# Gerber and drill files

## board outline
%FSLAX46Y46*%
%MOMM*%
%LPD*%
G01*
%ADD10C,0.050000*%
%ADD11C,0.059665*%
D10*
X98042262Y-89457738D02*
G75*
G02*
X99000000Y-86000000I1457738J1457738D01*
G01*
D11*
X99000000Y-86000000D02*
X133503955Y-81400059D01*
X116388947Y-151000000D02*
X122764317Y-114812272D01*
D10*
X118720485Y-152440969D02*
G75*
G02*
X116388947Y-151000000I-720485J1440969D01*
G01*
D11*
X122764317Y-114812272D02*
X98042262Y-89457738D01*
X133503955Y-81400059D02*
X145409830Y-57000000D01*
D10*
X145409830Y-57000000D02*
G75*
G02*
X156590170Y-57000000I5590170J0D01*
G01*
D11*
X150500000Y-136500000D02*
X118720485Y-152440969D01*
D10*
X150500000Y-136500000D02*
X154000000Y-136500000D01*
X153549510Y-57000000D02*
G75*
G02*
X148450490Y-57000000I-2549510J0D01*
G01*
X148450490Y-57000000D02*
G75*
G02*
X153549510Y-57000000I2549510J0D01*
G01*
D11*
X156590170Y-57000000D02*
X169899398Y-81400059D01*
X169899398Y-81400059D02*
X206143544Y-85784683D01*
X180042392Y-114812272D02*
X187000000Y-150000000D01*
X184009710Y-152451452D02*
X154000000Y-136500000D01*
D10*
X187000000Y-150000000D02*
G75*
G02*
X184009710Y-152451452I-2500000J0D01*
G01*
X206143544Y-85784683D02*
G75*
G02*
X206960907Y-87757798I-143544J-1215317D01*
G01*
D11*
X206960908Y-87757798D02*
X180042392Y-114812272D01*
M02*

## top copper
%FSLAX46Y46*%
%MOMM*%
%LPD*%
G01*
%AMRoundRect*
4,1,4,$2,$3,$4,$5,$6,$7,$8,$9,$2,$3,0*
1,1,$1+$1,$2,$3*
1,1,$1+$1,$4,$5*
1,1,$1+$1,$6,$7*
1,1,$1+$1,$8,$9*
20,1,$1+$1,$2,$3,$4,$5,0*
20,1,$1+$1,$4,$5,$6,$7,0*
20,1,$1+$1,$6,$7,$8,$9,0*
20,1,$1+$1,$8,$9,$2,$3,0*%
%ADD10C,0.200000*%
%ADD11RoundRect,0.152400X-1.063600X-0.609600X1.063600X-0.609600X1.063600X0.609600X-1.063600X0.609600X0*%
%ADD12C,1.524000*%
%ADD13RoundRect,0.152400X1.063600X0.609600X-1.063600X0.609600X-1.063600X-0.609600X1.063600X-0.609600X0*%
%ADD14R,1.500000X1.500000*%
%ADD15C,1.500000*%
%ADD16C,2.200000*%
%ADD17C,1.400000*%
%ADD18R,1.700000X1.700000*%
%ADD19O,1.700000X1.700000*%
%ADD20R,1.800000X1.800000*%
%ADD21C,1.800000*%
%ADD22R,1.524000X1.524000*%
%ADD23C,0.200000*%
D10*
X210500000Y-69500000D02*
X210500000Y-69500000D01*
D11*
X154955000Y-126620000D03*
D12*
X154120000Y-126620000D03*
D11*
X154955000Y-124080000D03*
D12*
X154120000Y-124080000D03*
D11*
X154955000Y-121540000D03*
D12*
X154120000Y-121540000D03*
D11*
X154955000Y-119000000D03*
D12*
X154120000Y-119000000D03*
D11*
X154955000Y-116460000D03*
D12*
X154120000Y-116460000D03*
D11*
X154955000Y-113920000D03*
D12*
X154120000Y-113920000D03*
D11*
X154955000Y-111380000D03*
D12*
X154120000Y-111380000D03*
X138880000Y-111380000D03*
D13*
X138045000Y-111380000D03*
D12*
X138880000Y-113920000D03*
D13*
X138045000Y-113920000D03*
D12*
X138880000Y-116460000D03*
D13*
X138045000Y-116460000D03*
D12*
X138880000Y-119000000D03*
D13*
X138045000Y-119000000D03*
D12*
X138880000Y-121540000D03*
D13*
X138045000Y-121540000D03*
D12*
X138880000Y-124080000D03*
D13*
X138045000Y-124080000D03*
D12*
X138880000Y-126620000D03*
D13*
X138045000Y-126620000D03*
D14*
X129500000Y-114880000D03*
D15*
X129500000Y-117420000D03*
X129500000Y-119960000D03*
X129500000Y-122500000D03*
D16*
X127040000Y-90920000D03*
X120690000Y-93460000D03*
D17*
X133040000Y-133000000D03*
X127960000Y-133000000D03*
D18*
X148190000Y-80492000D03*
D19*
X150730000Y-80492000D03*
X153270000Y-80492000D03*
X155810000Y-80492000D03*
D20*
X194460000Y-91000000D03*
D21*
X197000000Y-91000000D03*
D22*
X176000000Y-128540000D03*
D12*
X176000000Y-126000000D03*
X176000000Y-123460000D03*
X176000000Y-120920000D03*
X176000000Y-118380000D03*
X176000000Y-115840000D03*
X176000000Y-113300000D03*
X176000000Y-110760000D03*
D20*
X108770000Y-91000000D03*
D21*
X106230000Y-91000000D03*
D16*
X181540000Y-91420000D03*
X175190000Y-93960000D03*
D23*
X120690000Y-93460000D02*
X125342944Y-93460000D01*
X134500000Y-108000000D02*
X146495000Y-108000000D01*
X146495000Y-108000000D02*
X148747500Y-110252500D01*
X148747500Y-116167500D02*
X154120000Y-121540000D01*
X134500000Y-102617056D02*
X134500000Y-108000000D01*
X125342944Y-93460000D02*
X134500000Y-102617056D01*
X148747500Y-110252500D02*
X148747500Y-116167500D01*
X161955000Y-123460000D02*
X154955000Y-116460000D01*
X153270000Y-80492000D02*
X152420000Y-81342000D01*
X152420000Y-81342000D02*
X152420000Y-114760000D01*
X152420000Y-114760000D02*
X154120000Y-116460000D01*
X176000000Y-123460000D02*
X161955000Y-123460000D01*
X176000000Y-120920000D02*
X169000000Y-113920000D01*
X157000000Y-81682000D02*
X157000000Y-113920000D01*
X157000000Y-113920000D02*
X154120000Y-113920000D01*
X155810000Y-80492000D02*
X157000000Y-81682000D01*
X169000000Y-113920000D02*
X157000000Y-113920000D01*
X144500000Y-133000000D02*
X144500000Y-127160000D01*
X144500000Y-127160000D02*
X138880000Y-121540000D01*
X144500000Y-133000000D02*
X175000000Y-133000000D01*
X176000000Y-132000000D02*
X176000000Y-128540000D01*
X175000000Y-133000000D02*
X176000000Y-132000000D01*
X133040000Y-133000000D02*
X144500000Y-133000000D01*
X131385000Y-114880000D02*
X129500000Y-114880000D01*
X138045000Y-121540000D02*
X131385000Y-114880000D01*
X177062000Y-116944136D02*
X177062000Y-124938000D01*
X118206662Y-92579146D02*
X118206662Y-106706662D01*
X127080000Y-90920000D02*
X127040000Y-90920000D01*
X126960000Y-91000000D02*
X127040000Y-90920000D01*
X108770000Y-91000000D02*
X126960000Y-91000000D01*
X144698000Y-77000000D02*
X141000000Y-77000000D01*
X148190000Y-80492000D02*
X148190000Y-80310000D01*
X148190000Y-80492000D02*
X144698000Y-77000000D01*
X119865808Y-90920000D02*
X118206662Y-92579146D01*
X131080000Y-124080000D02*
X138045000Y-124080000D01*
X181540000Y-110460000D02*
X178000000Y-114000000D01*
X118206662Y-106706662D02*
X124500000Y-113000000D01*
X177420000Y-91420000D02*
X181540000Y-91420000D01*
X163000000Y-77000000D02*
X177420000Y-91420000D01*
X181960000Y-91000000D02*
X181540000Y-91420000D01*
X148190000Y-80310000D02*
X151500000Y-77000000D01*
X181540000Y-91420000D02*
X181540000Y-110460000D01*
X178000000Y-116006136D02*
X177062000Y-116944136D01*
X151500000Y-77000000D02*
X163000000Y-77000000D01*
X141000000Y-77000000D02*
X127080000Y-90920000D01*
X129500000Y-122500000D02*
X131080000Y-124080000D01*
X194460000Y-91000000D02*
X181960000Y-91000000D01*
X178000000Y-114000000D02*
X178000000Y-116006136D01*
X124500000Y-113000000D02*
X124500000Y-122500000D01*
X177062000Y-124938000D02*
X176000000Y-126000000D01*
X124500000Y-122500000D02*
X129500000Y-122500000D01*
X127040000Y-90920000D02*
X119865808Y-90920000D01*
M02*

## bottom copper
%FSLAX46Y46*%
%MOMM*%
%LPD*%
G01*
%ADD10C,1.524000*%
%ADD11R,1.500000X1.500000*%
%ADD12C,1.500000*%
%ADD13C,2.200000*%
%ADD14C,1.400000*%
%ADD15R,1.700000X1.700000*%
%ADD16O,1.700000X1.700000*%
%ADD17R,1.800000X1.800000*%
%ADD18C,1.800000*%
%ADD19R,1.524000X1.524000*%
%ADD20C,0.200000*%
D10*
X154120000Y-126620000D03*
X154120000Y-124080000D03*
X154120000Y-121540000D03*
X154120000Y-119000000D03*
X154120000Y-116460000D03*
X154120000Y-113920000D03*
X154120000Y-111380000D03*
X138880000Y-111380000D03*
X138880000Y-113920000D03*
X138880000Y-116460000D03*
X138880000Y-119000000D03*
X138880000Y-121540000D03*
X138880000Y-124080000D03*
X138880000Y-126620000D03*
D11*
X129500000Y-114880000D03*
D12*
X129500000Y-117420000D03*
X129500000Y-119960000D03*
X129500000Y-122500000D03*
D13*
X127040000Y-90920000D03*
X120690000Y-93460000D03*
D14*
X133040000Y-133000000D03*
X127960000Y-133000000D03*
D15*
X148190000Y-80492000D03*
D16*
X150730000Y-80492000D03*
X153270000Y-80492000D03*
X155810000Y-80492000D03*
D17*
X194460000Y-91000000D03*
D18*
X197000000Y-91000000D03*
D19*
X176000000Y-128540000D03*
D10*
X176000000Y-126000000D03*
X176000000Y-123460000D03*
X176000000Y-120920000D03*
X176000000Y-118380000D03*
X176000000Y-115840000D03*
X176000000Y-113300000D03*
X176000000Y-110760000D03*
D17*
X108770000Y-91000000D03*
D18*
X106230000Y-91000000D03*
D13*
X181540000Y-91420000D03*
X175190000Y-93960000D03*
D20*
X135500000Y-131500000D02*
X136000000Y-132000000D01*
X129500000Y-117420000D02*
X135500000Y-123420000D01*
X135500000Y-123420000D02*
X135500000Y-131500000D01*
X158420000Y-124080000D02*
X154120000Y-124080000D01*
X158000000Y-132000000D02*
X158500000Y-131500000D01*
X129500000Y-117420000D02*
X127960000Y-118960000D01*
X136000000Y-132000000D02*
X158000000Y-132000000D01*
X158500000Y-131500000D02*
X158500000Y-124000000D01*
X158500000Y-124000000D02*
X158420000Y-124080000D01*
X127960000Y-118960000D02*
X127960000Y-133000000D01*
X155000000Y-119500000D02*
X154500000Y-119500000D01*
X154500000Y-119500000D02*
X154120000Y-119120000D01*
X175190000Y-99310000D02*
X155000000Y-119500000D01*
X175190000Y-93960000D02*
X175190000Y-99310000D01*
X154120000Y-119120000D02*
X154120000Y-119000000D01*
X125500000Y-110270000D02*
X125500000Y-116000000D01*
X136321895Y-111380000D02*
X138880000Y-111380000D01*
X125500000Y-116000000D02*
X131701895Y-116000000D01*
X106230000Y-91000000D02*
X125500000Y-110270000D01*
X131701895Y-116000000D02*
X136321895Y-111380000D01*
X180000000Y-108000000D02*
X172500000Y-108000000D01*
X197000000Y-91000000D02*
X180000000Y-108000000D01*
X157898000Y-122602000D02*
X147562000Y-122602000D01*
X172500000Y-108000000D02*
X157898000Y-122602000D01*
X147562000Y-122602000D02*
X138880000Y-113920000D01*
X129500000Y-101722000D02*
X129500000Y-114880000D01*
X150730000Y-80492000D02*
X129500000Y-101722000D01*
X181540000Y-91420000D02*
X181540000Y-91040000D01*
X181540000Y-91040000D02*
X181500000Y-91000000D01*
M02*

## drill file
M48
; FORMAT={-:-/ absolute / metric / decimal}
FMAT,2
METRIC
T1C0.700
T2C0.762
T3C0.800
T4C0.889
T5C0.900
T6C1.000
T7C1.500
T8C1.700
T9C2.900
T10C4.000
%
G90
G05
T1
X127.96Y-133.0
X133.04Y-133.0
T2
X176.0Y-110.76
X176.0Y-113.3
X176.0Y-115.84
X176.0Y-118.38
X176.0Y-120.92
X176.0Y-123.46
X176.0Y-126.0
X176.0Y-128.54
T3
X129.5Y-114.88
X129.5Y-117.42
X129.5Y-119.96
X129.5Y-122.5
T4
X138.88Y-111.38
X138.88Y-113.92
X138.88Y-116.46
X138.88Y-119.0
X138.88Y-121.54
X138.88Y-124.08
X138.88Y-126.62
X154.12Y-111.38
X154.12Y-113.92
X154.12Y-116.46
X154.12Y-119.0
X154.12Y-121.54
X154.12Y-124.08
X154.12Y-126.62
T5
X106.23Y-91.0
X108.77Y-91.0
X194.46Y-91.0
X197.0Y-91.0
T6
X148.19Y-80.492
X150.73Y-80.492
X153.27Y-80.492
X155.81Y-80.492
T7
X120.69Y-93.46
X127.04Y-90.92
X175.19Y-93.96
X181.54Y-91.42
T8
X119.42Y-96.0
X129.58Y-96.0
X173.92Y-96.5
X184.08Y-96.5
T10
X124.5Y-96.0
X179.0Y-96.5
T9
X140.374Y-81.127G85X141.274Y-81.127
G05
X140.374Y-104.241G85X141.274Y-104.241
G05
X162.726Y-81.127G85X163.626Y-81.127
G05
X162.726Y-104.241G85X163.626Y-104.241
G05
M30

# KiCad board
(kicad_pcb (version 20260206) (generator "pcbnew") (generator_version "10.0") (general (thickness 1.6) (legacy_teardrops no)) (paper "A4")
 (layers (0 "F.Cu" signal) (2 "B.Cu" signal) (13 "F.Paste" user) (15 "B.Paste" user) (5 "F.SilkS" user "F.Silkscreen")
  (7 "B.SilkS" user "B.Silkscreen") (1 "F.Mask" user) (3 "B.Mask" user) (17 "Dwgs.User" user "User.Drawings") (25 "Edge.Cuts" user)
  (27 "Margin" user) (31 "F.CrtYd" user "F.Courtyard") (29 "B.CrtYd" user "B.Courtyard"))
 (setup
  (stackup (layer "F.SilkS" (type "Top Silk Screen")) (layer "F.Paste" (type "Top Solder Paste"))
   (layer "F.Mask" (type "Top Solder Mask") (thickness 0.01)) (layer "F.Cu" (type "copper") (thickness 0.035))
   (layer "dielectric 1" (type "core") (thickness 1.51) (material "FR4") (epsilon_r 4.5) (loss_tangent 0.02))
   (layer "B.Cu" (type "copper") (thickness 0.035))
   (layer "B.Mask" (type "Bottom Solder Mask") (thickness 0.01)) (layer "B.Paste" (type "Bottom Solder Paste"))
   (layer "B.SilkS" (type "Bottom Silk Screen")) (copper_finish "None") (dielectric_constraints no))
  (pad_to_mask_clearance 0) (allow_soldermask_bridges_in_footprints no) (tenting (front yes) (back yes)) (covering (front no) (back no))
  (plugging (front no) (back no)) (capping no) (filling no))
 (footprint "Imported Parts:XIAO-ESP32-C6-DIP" (layer "F.Cu") (at 146.5 119 -90)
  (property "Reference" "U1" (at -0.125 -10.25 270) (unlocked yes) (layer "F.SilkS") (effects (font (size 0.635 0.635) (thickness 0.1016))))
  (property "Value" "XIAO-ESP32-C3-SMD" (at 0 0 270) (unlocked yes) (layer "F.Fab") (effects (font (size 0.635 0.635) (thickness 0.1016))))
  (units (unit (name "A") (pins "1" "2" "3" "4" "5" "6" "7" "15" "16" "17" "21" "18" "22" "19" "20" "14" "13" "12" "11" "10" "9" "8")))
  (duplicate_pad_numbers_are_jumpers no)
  (pad "1" smd roundrect (at 7.62 -8.455) (size 2.432 1.524) (layers "F.Cu" "F.Mask") (roundrect_rratio 0.1)
   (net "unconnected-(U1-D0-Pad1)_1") (thermal_bridge_angle 45))
  (pad "1" thru_hole circle (at 7.62 -7.62) (size 1.524 1.524) (drill 0.889) (layers "*.Cu" "*.Mask") (remove_unused_layers no)
   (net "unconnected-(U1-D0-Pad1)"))
  (pad "2" smd roundrect (at 5.08 -8.455) (size 2.432 1.524) (layers "F.Cu" "F.Mask") (roundrect_rratio 0.1) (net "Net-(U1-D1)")
   (thermal_bridge_angle 45))
  (pad "2" thru_hole circle (at 5.08 -7.62) (size 1.524 1.524) (drill 0.889) (layers "*.Cu" "*.Mask") (remove_unused_layers no)
   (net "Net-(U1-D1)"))
  (pad "3" smd roundrect (at 2.54 -8.455) (size 2.432 1.524) (layers "F.Cu" "F.Mask") (roundrect_rratio 0.1) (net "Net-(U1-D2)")
   (thermal_bridge_angle 45))
  (pad "3" thru_hole circle (at 2.54 -7.62) (size 1.524 1.524) (drill 0.889) (layers "*.Cu" "*.Mask") (remove_unused_layers no)
   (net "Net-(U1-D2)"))
  (pad "4" smd roundrect (at 0 -8.455) (size 2.432 1.524) (layers "F.Cu" "F.Mask") (roundrect_rratio 0.1) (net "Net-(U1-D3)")
   (thermal_bridge_angle 45))
  (pad "4" thru_hole circle (at 0 -7.62) (size 1.524 1.524) (drill 0.889) (layers "*.Cu" "*.Mask") (remove_unused_layers no)
   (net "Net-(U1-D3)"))
  (pad "5" smd roundrect (at -2.54 -8.455) (size 2.432 1.524) (layers "F.Cu" "F.Mask") (roundrect_rratio 0.1) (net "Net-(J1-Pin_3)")
   (thermal_bridge_angle 45))
  (pad "5" thru_hole circle (at -2.54 -7.62) (size 1.524 1.524) (drill 0.889) (layers "*.Cu" "*.Mask") (remove_unused_layers no)
   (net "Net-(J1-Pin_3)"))
  (pad "6" smd roundrect (at -5.08 -8.455) (size 2.432 1.524) (layers "F.Cu" "F.Mask") (roundrect_rratio 0.1) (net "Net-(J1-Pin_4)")
   (thermal_bridge_angle 45))
  (pad "6" thru_hole circle (at -5.08 -7.62) (size 1.524 1.524) (drill 0.889) (layers "*.Cu" "*.Mask") (remove_unused_layers no)
   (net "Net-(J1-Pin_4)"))
  (pad "7" smd roundrect (at -7.62 -8.455) (size 2.432 1.524) (layers "F.Cu" "F.Mask") (roundrect_rratio 0.1)
   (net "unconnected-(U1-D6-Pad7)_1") (thermal_bridge_angle 45))
  (pad "7" thru_hole circle (at -7.62 -7.62) (size 1.524 1.524) (drill 0.889) (layers "*.Cu" "*.Mask") (remove_unused_layers no)
   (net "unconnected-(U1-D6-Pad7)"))
  (pad "8" thru_hole circle (at -7.62 7.62 180) (size 1.524 1.524) (drill 0.889) (layers "*.Cu" "*.Mask") (remove_unused_layers no)
   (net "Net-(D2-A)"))
  (pad "8" smd roundrect (at -7.62 8.455 180) (size 2.432 1.524) (layers "F.Cu" "F.Mask") (roundrect_rratio 0.1) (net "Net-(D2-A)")
   (thermal_bridge_angle 45))
  (pad "9" thru_hole circle (at -5.08 7.62 180) (size 1.524 1.524) (drill 0.889) (layers "*.Cu" "*.Mask") (remove_unused_layers no)
   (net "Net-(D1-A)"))
  (pad "9" smd roundrect (at -5.08 8.455 180) (size 2.432 1.524) (layers "F.Cu" "F.Mask") (roundrect_rratio 0.1) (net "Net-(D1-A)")
   (thermal_bridge_angle 45))
  (pad "10" thru_hole circle (at -2.54 7.62 180) (size 1.524 1.524) (drill 0.889) (layers "*.Cu" "*.Mask") (remove_unused_layers no)
   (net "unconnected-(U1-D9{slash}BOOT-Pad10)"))
  (pad "10" smd roundrect (at -2.54 8.455 180) (size 2.432 1.524) (layers "F.Cu" "F.Mask") (roundrect_rratio 0.1)
   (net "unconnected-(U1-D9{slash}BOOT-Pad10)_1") (thermal_bridge_angle 45))
  (pad "11" thru_hole circle (at 0 7.62 180) (size 1.524 1.524) (drill 0.889) (layers "*.Cu" "*.Mask") (remove_unused_layers no)
   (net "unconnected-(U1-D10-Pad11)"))
  (pad "11" smd roundrect (at 0 8.455 180) (size 2.432 1.524) (layers "F.Cu" "F.Mask") (roundrect_rratio 0.1)
   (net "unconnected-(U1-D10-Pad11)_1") (thermal_bridge_angle 45))
  (pad "12" thru_hole circle (at 2.54 7.62 180) (size 1.524 1.524) (drill 0.889) (layers "*.Cu" "*.Mask") (remove_unused_layers no)
   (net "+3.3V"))
  (pad "12" smd roundrect (at 2.54 8.455 180) (size 2.432 1.524) (layers "F.Cu" "F.Mask") (roundrect_rratio 0.1) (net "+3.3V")
   (thermal_bridge_angle 45))
  (pad "13" thru_hole circle (at 5.08 7.62 180) (size 1.524 1.524) (drill 0.889) (layers "*.Cu" "*.Mask") (remove_unused_layers no)
   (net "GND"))
  (pad "13" smd roundrect (at 5.08 8.455 180) (size 2.432 1.524) (layers "F.Cu" "F.Mask") (roundrect_rratio 0.1) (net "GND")
   (thermal_bridge_angle 45))
  (pad "14" thru_hole circle (at 7.62 7.62 180) (size 1.524 1.524) (drill 0.889) (layers "*.Cu" "*.Mask") (remove_unused_layers no)
   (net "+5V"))
  (pad "14" smd roundrect (at 7.62 8.455 180) (size 2.432 1.524) (layers "F.Cu" "F.Mask") (roundrect_rratio 0.1) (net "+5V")
   (thermal_bridge_angle 45)))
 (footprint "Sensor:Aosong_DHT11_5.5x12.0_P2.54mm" (layer "F.Cu") (at 129.5 114.88)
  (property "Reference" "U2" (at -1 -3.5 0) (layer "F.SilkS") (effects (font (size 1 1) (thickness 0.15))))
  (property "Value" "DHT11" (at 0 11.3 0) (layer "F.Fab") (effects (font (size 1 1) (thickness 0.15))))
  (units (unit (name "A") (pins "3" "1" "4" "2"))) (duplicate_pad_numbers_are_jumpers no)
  (pad "1" thru_hole rect (at 0 0) (size 1.5 1.5) (drill 0.8) (layers "*.Cu" "*.Mask") (remove_unused_layers no) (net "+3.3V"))
  (pad "2" thru_hole circle (at 0 2.54) (size 1.5 1.5) (drill 0.8) (layers "*.Cu" "*.Mask") (remove_unused_layers no) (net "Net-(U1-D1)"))
  (pad "3" thru_hole circle (at 0 5.08) (size 1.5 1.5) (drill 0.8) (layers "*.Cu" "*.Mask") (remove_unused_layers no)
   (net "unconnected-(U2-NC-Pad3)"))
  (pad "4" thru_hole circle (at 0 7.62) (size 1.5 1.5) (drill 0.8) (layers "*.Cu" "*.Mask") (remove_unused_layers no) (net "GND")))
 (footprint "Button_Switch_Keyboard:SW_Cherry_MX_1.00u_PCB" (layer "F.Cu") (at 127.04 90.92)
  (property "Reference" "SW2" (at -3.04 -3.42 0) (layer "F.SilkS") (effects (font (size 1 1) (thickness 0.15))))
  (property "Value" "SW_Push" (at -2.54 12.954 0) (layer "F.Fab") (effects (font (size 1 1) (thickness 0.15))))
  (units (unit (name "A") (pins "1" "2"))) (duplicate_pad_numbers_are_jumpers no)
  (pad "" np_thru_hole circle (at -7.62 5.08) (size 1.7 1.7) (drill 1.7) (layers "*.Cu" "*.Mask"))
  (pad "" np_thru_hole circle (at -2.54 5.08) (size 4 4) (drill 4) (layers "*.Cu" "*.Mask"))
  (pad "" np_thru_hole circle (at 2.54 5.08) (size 1.7 1.7) (drill 1.7) (layers "*.Cu" "*.Mask"))
  (pad "1" thru_hole circle (at 0 0) (size 2.2 2.2) (drill 1.5) (layers "*.Cu" "*.Mask") (remove_unused_layers no) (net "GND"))
  (pad "2" thru_hole circle (at -6.35 2.54) (size 2.2 2.2) (drill 1.5) (layers "*.Cu" "*.Mask") (remove_unused_layers no)
   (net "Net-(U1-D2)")))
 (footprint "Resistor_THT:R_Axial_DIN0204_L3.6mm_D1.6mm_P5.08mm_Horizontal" (layer "F.Cu") (at 133.04 133 180)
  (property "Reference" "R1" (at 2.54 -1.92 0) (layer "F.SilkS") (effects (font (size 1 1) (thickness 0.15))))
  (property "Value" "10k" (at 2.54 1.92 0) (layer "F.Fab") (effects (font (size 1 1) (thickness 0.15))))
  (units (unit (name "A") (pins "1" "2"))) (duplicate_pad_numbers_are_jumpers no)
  (pad "1" thru_hole circle (at 0 0 180) (size 1.4 1.4) (drill 0.7) (layers "*.Cu" "*.Mask") (remove_unused_layers no) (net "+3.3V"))
  (pad "2" thru_hole circle (at 5.08 0 180) (size 1.4 1.4) (drill 0.7) (layers "*.Cu" "*.Mask") (remove_unused_layers no)
   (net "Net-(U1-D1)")))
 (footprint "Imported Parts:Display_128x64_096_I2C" (layer "F.Cu") (at 152 80.492)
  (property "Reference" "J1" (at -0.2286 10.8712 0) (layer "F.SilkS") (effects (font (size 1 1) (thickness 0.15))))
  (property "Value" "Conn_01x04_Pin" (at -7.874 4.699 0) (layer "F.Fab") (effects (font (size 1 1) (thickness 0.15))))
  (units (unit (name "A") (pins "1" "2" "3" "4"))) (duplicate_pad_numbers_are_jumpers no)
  (pad "" np_thru_hole oval (at -11.176 0.635) (size 3.8 2.9) (drill oval 3.8 2.9) (layers "*.Cu" "*.Mask"))
  (pad "" np_thru_hole oval (at -11.176 23.749) (size 3.8 2.9) (drill oval 3.8 2.9) (layers "*.Cu" "*.Mask"))
  (pad "" np_thru_hole oval (at 11.176 0.635) (size 3.8 2.9) (drill oval 3.8 2.9) (layers "*.Cu" "*.Mask"))
  (pad "" np_thru_hole oval (at 11.176 23.749) (size 3.8 2.9) (drill oval 3.8 2.9) (layers "*.Cu" "*.Mask"))
  (pad "1" thru_hole rect (at -3.81 0 90) (size 1.7 1.7) (drill 1) (layers "*.Cu" "*.Mask") (remove_unused_layers no) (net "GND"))
  (pad "2" thru_hole oval (at -1.27 0 90) (size 1.7 1.7) (drill 1) (layers "*.Cu" "*.Mask") (remove_unused_layers no) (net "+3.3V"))
  (pad "3" thru_hole oval (at 1.27 0 90) (size 1.7 1.7) (drill 1) (layers "*.Cu" "*.Mask") (remove_unused_layers no) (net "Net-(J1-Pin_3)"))
  (pad "4" thru_hole oval (at 3.81 0 90) (size 1.7 1.7) (drill 1) (layers "*.Cu" "*.Mask") (remove_unused_layers no) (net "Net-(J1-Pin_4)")))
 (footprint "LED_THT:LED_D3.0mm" (layer "F.Cu") (at 194.46 91)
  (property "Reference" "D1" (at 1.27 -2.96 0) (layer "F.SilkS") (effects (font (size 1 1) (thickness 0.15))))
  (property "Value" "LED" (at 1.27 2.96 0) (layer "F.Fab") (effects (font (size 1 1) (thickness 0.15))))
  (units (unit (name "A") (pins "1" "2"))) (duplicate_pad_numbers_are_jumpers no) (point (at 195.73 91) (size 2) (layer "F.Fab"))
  (pad "1" thru_hole rect (at 0 0) (size 1.8 1.8) (drill 0.9) (layers "*.Cu" "*.Mask") (remove_unused_layers no) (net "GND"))
  (pad "2" thru_hole circle (at 2.54 0) (size 1.8 1.8) (drill 0.9) (layers "*.Cu" "*.Mask") (remove_unused_layers no) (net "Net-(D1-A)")))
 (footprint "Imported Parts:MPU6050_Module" (layer "F.Cu") (at 176 128.54 180)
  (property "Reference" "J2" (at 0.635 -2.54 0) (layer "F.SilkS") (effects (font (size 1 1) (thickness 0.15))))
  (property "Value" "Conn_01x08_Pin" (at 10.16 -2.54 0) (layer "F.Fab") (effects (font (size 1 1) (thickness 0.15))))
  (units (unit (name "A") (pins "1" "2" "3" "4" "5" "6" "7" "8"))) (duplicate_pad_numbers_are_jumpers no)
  (pad "1" thru_hole rect (at 0 0 180) (size 1.524 1.524) (drill 0.762) (layers "*.Cu" "*.Mask") (remove_unused_layers no) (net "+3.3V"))
  (pad "2" thru_hole circle (at 0 2.54 180) (size 1.524 1.524) (drill 0.762) (layers "*.Cu" "*.Mask") (remove_unused_layers no) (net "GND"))
  (pad "3" thru_hole circle (at 0 5.08 180) (size 1.524 1.524) (drill 0.762) (layers "*.Cu" "*.Mask") (remove_unused_layers no)
   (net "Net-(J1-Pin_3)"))
  (pad "4" thru_hole circle (at 0 7.62 180) (size 1.524 1.524) (drill 0.762) (layers "*.Cu" "*.Mask") (remove_unused_layers no)
   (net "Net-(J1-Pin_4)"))
  (pad "5" thru_hole circle (at 0 10.16 180) (size 1.524 1.524) (drill 0.762) (layers "*.Cu" "*.Mask") (remove_unused_layers no)
   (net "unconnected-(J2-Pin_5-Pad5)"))
  (pad "6" thru_hole circle (at 0 12.7 180) (size 1.524 1.524) (drill 0.762) (layers "*.Cu" "*.Mask") (remove_unused_layers no)
   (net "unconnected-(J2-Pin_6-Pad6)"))
  (pad "7" thru_hole circle (at 0 15.24 180) (size 1.524 1.524) (drill 0.762) (layers "*.Cu" "*.Mask") (remove_unused_layers no)
   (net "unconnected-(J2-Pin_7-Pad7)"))
  (pad "8" thru_hole circle (at 0 17.78 180) (size 1.524 1.524) (drill 0.762) (layers "*.Cu" "*.Mask") (remove_unused_layers no)
   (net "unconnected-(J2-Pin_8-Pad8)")))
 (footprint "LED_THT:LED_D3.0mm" (layer "F.Cu") (at 108.77 91 180)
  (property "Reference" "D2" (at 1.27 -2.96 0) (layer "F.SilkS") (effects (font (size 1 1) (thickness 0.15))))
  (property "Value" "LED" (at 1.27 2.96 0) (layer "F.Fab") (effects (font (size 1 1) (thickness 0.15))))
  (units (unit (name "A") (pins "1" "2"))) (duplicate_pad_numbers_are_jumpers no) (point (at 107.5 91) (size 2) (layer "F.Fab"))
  (pad "1" thru_hole rect (at 0 0 180) (size 1.8 1.8) (drill 0.9) (layers "*.Cu" "*.Mask") (remove_unused_layers no) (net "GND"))
  (pad "2" thru_hole circle (at 2.54 0 180) (size 1.8 1.8) (drill 0.9) (layers "*.Cu" "*.Mask") (remove_unused_layers no) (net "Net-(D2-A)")))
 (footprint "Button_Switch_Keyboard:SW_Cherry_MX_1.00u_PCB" (layer "F.Cu") (at 181.54 91.42)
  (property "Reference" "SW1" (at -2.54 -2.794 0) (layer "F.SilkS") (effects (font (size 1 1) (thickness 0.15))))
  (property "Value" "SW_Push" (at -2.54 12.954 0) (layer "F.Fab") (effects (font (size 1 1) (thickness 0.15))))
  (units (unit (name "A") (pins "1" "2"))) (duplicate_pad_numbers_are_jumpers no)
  (pad "" np_thru_hole circle (at -7.62 5.08) (size 1.7 1.7) (drill 1.7) (layers "*.Cu" "*.Mask"))
  (pad "" np_thru_hole circle (at -2.54 5.08) (size 4 4) (drill 4) (layers "*.Cu" "*.Mask"))
  (pad "" np_thru_hole circle (at 2.54 5.08) (size 1.7 1.7) (drill 1.7) (layers "*.Cu" "*.Mask"))
  (pad "1" thru_hole circle (at 0 0) (size 2.2 2.2) (drill 1.5) (layers "*.Cu" "*.Mask") (remove_unused_layers no) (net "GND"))
  (pad "2" thru_hole circle (at -6.35 2.54) (size 2.2 2.2) (drill 1.5) (layers "*.Cu" "*.Mask") (remove_unused_layers no)
   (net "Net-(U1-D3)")))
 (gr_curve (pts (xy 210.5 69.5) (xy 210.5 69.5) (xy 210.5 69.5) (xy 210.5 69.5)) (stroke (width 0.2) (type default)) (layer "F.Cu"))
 (gr_arc (start 98.042262 89.457738) (mid 97.513251 87.449702) (end 99 86) (stroke (width 0.05) (type default)) (layer "Edge.Cuts"))
 (gr_line (start 99 86) (end 133.503955 81.400059) (stroke (width 0.059665) (type default)) (layer "Edge.Cuts"))
 (gr_line (start 116.388947 151) (end 122.764317 114.812272) (stroke (width 0.059665) (type default)) (layer "Edge.Cuts"))
 (gr_arc (start 118.720485 152.440969) (mid 117.15302 152.370443) (end 116.388947 151) (stroke (width 0.05) (type default))
  (layer "Edge.Cuts"))
 (gr_line (start 122.764317 114.812272) (end 98.042262 89.457738) (stroke (width 0.059665) (type default)) (layer "Edge.Cuts"))
 (gr_line (start 133.503955 81.400059) (end 145.40983 57) (stroke (width 0.059665) (type default)) (layer "Edge.Cuts"))
 (gr_arc (start 145.40983 57) (mid 151 51.40983) (end 156.59017 57) (stroke (width 0.05) (type default)) (layer "Edge.Cuts"))
 (gr_line (start 150.5 136.5) (end 118.720485 152.440969) (stroke (width 0.059665) (type default)) (layer "Edge.Cuts"))
 (gr_line (start 150.5 136.5) (end 154 136.5) (stroke (width 0.05) (type default)) (layer "Edge.Cuts"))
 (gr_circle (center 151 57) (end 151.5 54.5) (stroke (width 0.05) (type default)) (fill no) (layer "Edge.Cuts"))
 (gr_line (start 156.59017 57) (end 169.899398 81.400059) (stroke (width 0.059665) (type default)) (layer "Edge.Cuts"))
 (gr_line (start 169.899398 81.400059) (end 206.143544 85.784683) (stroke (width 0.059665) (type default)) (layer "Edge.Cuts"))
 (gr_line (start 180.042392 114.812272) (end 187 150) (stroke (width 0.059665) (type default)) (layer "Edge.Cuts"))
 (gr_line (start 184.00971 152.451452) (end 154 136.5) (stroke (width 0.059665) (type default)) (layer "Edge.Cuts"))
 (gr_arc (start 187 150) (mid 186.084972 151.933355) (end 184.00971 152.451452) (stroke (width 0.05) (type default)) (layer "Edge.Cuts"))
 (gr_arc (start 206.143544 85.784683) (mid 207.130597 86.53165) (end 206.960908 87.757798) (stroke (width 0.05) (type default))
  (layer "Edge.Cuts"))
 (gr_line (start 206.960908 87.757798) (end 180.042392 114.812272) (stroke (width 0.059665) (type default)) (layer "Edge.Cuts"))
 (segment (start 135.5 131.5) (end 136 132) (width 0.2) (layer "B.Cu") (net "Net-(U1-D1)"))
 (segment (start 129.5 117.42) (end 135.5 123.42) (width 0.2) (layer "B.Cu") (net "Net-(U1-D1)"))
 (segment (start 135.5 123.42) (end 135.5 131.5) (width 0.2) (layer "B.Cu") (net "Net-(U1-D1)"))
 (segment (start 158.42 124.08) (end 154.12 124.08) (width 0.2) (layer "B.Cu") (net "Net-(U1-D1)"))
 (segment (start 158 132) (end 158.5 131.5) (width 0.2) (layer "B.Cu") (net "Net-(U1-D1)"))
 (segment (start 129.5 117.42) (end 127.96 118.96) (width 0.2) (layer "B.Cu") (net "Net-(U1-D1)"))
 (segment (start 136 132) (end 158 132) (width 0.2) (layer "B.Cu") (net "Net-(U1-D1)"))
 (segment (start 158.5 131.5) (end 158.5 124) (width 0.2) (layer "B.Cu") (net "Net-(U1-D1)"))
 (segment (start 158.5 124) (end 158.42 124.08) (width 0.2) (layer "B.Cu") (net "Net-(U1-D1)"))
 (segment (start 127.96 118.96) (end 127.96 133) (width 0.2) (layer "B.Cu") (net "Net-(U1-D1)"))
 (segment (start 120.69 93.46) (end 125.342944 93.46) (width 0.2) (layer "F.Cu") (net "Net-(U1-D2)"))
 (segment (start 134.5 108) (end 146.495 108) (width 0.2) (layer "F.Cu") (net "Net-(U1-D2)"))
 (segment (start 146.495 108) (end 148.7475 110.2525) (width 0.2) (layer "F.Cu") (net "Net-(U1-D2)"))
 (segment (start 148.7475 116.1675) (end 154.12 121.54) (width 0.2) (layer "F.Cu") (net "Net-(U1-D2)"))
 (segment (start 134.5 102.617056) (end 134.5 108) (width 0.2) (layer "F.Cu") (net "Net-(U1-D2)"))
 (segment (start 125.342944 93.46) (end 134.5 102.617056) (width 0.2) (layer "F.Cu") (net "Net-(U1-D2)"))
 (segment (start 148.7475 110.2525) (end 148.7475 116.1675) (width 0.2) (layer "F.Cu") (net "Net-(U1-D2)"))
 (segment (start 155 119.5) (end 154.5 119.5) (width 0.2) (layer "B.Cu") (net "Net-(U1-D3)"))
 (segment (start 154.5 119.5) (end 154.12 119.12) (width 0.2) (layer "B.Cu") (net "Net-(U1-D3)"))
 (segment (start 175.19 99.31) (end 155 119.5) (width 0.2) (layer "B.Cu") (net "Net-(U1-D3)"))
 (segment (start 175.19 93.96) (end 175.19 99.31) (width 0.2) (layer "B.Cu") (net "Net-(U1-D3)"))
 (segment (start 154.12 119.12) (end 154.12 119) (width 0.2) (layer "B.Cu") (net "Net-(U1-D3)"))
 (segment (start 161.955 123.46) (end 154.955 116.46) (width 0.2) (layer "F.Cu") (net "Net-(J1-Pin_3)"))
 (segment (start 153.27 80.492) (end 152.42 81.342) (width 0.2) (layer "F.Cu") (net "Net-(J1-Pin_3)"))
 (segment (start 152.42 81.342) (end 152.42 114.76) (width 0.2) (layer "F.Cu") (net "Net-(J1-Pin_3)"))
 (segment (start 152.42 114.76) (end 154.12 116.46) (width 0.2) (layer "F.Cu") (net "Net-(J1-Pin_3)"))
 (segment (start 176 123.46) (end 161.955 123.46) (width 0.2) (layer "F.Cu") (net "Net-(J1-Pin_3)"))
 (segment (start 176 120.92) (end 169 113.92) (width 0.2) (layer "F.Cu") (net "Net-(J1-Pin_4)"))
 (segment (start 157 81.682) (end 157 113.92) (width 0.2) (layer "F.Cu") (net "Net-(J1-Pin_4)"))
 (segment (start 157 113.92) (end 154.12 113.92) (width 0.2) (layer "F.Cu") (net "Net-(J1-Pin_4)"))
 (segment (start 155.81 80.492) (end 157 81.682) (width 0.2) (layer "F.Cu") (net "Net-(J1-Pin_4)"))
 (segment (start 169 113.92) (end 157 113.92) (width 0.2) (layer "F.Cu") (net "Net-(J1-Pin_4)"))
 (segment (start 125.5 110.27) (end 125.5 116) (width 0.2) (layer "B.Cu") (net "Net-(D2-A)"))
 (segment (start 136.321895 111.38) (end 138.88 111.38) (width 0.2) (layer "B.Cu") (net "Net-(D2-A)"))
 (segment (start 125.5 116) (end 131.701895 116) (width 0.2) (layer "B.Cu") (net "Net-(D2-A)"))
 (segment (start 106.23 91) (end 125.5 110.27) (width 0.2) (layer "B.Cu") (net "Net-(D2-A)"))
 (segment (start 131.701895 116) (end 136.321895 111.38) (width 0.2) (layer "B.Cu") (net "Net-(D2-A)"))
 (segment (start 180 108) (end 172.5 108) (width 0.2) (layer "B.Cu") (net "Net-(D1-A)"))
 (segment (start 197 91) (end 180 108) (width 0.2) (layer "B.Cu") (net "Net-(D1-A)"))
 (segment (start 157.898 122.602) (end 147.562 122.602) (width 0.2) (layer "B.Cu") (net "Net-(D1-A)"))
 (segment (start 172.5 108) (end 157.898 122.602) (width 0.2) (layer "B.Cu") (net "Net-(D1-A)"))
 (segment (start 147.562 122.602) (end 138.88 113.92) (width 0.2) (layer "B.Cu") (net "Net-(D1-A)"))
 (segment (start 144.5 133) (end 144.5 127.16) (width 0.2) (layer "F.Cu") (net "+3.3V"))
 (segment (start 144.5 127.16) (end 138.88 121.54) (width 0.2) (layer "F.Cu") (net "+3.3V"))
 (segment (start 144.5 133) (end 175 133) (width 0.2) (layer "F.Cu") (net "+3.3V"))
 (segment (start 176 132) (end 176 128.54) (width 0.2) (layer "F.Cu") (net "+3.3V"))
 (segment (start 175 133) (end 176 132) (width 0.2) (layer "F.Cu") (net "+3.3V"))
 (segment (start 133.04 133) (end 144.5 133) (width 0.2) (layer "F.Cu") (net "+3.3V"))
 (segment (start 131.385 114.88) (end 129.5 114.88) (width 0.2) (layer "F.Cu") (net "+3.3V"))
 (segment (start 138.045 121.54) (end 131.385 114.88) (width 0.2) (layer "F.Cu") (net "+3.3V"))
 (segment (start 129.5 101.722) (end 129.5 114.88) (width 0.2) (layer "B.Cu") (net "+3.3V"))
 (segment (start 150.73 80.492) (end 129.5 101.722) (width 0.2) (layer "B.Cu") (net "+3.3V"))
 (segment (start 177.062 116.944136) (end 177.062 124.938) (width 0.2) (layer "F.Cu") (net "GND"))
 (segment (start 118.206662 92.579146) (end 118.206662 106.706662) (width 0.2) (layer "F.Cu") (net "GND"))
 (segment (start 127.08 90.92) (end 127.04 90.92) (width 0.2) (layer "F.Cu") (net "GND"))
 (segment (start 126.96 91) (end 127.04 90.92) (width 0.2) (layer "F.Cu") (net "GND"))
 (segment (start 108.77 91) (end 126.96 91) (width 0.2) (layer "F.Cu") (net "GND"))
 (segment (start 144.698 77) (end 141 77) (width 0.2) (layer "F.Cu") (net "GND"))
 (segment (start 148.19 80.492) (end 148.19 80.31) (width 0.2) (layer "F.Cu") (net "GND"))
 (segment (start 148.19 80.492) (end 144.698 77) (width 0.2) (layer "F.Cu") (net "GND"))
 (segment (start 119.865808 90.92) (end 118.206662 92.579146) (width 0.2) (layer "F.Cu") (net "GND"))
 (segment (start 131.08 124.08) (end 138.045 124.08) (width 0.2) (layer "F.Cu") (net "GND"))
 (segment (start 181.54 110.46) (end 178 114) (width 0.2) (layer "F.Cu") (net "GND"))
 (segment (start 118.206662 106.706662) (end 124.5 113) (width 0.2) (layer "F.Cu") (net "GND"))
 (segment (start 177.42 91.42) (end 181.54 91.42) (width 0.2) (layer "F.Cu") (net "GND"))
 (segment (start 163 77) (end 177.42 91.42) (width 0.2) (layer "F.Cu") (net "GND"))
 (segment (start 181.96 91) (end 181.54 91.42) (width 0.2) (layer "F.Cu") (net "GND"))
 (segment (start 148.19 80.31) (end 151.5 77) (width 0.2) (layer "F.Cu") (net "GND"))
 (segment (start 181.54 91.42) (end 181.54 110.46) (width 0.2) (layer "F.Cu") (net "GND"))
 (segment (start 178 116.006136) (end 177.062 116.944136) (width 0.2) (layer "F.Cu") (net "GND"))
 (segment (start 151.5 77) (end 163 77) (width 0.2) (layer "F.Cu") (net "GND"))
 (segment (start 141 77) (end 127.08 90.92) (width 0.2) (layer "F.Cu") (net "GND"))
 (segment (start 129.5 122.5) (end 131.08 124.08) (width 0.2) (layer "F.Cu") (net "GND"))
 (segment (start 194.46 91) (end 181.96 91) (width 0.2) (layer "F.Cu") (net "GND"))
 (segment (start 178 114) (end 178 116.006136) (width 0.2) (layer "F.Cu") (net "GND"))
 (segment (start 124.5 113) (end 124.5 122.5) (width 0.2) (layer "F.Cu") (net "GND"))
 (segment (start 177.062 124.938) (end 176 126) (width 0.2) (layer "F.Cu") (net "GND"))
 (segment (start 124.5 122.5) (end 129.5 122.5) (width 0.2) (layer "F.Cu") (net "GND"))
 (segment (start 127.04 90.92) (end 119.865808 90.92) (width 0.2) (layer "F.Cu") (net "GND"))
 (segment (start 181.54 91.42) (end 181.54 91.04) (width 0.2) (layer "B.Cu") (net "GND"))
 (segment (start 181.54 91.04) (end 181.5 91) (width 0.2) (layer "B.Cu") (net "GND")))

